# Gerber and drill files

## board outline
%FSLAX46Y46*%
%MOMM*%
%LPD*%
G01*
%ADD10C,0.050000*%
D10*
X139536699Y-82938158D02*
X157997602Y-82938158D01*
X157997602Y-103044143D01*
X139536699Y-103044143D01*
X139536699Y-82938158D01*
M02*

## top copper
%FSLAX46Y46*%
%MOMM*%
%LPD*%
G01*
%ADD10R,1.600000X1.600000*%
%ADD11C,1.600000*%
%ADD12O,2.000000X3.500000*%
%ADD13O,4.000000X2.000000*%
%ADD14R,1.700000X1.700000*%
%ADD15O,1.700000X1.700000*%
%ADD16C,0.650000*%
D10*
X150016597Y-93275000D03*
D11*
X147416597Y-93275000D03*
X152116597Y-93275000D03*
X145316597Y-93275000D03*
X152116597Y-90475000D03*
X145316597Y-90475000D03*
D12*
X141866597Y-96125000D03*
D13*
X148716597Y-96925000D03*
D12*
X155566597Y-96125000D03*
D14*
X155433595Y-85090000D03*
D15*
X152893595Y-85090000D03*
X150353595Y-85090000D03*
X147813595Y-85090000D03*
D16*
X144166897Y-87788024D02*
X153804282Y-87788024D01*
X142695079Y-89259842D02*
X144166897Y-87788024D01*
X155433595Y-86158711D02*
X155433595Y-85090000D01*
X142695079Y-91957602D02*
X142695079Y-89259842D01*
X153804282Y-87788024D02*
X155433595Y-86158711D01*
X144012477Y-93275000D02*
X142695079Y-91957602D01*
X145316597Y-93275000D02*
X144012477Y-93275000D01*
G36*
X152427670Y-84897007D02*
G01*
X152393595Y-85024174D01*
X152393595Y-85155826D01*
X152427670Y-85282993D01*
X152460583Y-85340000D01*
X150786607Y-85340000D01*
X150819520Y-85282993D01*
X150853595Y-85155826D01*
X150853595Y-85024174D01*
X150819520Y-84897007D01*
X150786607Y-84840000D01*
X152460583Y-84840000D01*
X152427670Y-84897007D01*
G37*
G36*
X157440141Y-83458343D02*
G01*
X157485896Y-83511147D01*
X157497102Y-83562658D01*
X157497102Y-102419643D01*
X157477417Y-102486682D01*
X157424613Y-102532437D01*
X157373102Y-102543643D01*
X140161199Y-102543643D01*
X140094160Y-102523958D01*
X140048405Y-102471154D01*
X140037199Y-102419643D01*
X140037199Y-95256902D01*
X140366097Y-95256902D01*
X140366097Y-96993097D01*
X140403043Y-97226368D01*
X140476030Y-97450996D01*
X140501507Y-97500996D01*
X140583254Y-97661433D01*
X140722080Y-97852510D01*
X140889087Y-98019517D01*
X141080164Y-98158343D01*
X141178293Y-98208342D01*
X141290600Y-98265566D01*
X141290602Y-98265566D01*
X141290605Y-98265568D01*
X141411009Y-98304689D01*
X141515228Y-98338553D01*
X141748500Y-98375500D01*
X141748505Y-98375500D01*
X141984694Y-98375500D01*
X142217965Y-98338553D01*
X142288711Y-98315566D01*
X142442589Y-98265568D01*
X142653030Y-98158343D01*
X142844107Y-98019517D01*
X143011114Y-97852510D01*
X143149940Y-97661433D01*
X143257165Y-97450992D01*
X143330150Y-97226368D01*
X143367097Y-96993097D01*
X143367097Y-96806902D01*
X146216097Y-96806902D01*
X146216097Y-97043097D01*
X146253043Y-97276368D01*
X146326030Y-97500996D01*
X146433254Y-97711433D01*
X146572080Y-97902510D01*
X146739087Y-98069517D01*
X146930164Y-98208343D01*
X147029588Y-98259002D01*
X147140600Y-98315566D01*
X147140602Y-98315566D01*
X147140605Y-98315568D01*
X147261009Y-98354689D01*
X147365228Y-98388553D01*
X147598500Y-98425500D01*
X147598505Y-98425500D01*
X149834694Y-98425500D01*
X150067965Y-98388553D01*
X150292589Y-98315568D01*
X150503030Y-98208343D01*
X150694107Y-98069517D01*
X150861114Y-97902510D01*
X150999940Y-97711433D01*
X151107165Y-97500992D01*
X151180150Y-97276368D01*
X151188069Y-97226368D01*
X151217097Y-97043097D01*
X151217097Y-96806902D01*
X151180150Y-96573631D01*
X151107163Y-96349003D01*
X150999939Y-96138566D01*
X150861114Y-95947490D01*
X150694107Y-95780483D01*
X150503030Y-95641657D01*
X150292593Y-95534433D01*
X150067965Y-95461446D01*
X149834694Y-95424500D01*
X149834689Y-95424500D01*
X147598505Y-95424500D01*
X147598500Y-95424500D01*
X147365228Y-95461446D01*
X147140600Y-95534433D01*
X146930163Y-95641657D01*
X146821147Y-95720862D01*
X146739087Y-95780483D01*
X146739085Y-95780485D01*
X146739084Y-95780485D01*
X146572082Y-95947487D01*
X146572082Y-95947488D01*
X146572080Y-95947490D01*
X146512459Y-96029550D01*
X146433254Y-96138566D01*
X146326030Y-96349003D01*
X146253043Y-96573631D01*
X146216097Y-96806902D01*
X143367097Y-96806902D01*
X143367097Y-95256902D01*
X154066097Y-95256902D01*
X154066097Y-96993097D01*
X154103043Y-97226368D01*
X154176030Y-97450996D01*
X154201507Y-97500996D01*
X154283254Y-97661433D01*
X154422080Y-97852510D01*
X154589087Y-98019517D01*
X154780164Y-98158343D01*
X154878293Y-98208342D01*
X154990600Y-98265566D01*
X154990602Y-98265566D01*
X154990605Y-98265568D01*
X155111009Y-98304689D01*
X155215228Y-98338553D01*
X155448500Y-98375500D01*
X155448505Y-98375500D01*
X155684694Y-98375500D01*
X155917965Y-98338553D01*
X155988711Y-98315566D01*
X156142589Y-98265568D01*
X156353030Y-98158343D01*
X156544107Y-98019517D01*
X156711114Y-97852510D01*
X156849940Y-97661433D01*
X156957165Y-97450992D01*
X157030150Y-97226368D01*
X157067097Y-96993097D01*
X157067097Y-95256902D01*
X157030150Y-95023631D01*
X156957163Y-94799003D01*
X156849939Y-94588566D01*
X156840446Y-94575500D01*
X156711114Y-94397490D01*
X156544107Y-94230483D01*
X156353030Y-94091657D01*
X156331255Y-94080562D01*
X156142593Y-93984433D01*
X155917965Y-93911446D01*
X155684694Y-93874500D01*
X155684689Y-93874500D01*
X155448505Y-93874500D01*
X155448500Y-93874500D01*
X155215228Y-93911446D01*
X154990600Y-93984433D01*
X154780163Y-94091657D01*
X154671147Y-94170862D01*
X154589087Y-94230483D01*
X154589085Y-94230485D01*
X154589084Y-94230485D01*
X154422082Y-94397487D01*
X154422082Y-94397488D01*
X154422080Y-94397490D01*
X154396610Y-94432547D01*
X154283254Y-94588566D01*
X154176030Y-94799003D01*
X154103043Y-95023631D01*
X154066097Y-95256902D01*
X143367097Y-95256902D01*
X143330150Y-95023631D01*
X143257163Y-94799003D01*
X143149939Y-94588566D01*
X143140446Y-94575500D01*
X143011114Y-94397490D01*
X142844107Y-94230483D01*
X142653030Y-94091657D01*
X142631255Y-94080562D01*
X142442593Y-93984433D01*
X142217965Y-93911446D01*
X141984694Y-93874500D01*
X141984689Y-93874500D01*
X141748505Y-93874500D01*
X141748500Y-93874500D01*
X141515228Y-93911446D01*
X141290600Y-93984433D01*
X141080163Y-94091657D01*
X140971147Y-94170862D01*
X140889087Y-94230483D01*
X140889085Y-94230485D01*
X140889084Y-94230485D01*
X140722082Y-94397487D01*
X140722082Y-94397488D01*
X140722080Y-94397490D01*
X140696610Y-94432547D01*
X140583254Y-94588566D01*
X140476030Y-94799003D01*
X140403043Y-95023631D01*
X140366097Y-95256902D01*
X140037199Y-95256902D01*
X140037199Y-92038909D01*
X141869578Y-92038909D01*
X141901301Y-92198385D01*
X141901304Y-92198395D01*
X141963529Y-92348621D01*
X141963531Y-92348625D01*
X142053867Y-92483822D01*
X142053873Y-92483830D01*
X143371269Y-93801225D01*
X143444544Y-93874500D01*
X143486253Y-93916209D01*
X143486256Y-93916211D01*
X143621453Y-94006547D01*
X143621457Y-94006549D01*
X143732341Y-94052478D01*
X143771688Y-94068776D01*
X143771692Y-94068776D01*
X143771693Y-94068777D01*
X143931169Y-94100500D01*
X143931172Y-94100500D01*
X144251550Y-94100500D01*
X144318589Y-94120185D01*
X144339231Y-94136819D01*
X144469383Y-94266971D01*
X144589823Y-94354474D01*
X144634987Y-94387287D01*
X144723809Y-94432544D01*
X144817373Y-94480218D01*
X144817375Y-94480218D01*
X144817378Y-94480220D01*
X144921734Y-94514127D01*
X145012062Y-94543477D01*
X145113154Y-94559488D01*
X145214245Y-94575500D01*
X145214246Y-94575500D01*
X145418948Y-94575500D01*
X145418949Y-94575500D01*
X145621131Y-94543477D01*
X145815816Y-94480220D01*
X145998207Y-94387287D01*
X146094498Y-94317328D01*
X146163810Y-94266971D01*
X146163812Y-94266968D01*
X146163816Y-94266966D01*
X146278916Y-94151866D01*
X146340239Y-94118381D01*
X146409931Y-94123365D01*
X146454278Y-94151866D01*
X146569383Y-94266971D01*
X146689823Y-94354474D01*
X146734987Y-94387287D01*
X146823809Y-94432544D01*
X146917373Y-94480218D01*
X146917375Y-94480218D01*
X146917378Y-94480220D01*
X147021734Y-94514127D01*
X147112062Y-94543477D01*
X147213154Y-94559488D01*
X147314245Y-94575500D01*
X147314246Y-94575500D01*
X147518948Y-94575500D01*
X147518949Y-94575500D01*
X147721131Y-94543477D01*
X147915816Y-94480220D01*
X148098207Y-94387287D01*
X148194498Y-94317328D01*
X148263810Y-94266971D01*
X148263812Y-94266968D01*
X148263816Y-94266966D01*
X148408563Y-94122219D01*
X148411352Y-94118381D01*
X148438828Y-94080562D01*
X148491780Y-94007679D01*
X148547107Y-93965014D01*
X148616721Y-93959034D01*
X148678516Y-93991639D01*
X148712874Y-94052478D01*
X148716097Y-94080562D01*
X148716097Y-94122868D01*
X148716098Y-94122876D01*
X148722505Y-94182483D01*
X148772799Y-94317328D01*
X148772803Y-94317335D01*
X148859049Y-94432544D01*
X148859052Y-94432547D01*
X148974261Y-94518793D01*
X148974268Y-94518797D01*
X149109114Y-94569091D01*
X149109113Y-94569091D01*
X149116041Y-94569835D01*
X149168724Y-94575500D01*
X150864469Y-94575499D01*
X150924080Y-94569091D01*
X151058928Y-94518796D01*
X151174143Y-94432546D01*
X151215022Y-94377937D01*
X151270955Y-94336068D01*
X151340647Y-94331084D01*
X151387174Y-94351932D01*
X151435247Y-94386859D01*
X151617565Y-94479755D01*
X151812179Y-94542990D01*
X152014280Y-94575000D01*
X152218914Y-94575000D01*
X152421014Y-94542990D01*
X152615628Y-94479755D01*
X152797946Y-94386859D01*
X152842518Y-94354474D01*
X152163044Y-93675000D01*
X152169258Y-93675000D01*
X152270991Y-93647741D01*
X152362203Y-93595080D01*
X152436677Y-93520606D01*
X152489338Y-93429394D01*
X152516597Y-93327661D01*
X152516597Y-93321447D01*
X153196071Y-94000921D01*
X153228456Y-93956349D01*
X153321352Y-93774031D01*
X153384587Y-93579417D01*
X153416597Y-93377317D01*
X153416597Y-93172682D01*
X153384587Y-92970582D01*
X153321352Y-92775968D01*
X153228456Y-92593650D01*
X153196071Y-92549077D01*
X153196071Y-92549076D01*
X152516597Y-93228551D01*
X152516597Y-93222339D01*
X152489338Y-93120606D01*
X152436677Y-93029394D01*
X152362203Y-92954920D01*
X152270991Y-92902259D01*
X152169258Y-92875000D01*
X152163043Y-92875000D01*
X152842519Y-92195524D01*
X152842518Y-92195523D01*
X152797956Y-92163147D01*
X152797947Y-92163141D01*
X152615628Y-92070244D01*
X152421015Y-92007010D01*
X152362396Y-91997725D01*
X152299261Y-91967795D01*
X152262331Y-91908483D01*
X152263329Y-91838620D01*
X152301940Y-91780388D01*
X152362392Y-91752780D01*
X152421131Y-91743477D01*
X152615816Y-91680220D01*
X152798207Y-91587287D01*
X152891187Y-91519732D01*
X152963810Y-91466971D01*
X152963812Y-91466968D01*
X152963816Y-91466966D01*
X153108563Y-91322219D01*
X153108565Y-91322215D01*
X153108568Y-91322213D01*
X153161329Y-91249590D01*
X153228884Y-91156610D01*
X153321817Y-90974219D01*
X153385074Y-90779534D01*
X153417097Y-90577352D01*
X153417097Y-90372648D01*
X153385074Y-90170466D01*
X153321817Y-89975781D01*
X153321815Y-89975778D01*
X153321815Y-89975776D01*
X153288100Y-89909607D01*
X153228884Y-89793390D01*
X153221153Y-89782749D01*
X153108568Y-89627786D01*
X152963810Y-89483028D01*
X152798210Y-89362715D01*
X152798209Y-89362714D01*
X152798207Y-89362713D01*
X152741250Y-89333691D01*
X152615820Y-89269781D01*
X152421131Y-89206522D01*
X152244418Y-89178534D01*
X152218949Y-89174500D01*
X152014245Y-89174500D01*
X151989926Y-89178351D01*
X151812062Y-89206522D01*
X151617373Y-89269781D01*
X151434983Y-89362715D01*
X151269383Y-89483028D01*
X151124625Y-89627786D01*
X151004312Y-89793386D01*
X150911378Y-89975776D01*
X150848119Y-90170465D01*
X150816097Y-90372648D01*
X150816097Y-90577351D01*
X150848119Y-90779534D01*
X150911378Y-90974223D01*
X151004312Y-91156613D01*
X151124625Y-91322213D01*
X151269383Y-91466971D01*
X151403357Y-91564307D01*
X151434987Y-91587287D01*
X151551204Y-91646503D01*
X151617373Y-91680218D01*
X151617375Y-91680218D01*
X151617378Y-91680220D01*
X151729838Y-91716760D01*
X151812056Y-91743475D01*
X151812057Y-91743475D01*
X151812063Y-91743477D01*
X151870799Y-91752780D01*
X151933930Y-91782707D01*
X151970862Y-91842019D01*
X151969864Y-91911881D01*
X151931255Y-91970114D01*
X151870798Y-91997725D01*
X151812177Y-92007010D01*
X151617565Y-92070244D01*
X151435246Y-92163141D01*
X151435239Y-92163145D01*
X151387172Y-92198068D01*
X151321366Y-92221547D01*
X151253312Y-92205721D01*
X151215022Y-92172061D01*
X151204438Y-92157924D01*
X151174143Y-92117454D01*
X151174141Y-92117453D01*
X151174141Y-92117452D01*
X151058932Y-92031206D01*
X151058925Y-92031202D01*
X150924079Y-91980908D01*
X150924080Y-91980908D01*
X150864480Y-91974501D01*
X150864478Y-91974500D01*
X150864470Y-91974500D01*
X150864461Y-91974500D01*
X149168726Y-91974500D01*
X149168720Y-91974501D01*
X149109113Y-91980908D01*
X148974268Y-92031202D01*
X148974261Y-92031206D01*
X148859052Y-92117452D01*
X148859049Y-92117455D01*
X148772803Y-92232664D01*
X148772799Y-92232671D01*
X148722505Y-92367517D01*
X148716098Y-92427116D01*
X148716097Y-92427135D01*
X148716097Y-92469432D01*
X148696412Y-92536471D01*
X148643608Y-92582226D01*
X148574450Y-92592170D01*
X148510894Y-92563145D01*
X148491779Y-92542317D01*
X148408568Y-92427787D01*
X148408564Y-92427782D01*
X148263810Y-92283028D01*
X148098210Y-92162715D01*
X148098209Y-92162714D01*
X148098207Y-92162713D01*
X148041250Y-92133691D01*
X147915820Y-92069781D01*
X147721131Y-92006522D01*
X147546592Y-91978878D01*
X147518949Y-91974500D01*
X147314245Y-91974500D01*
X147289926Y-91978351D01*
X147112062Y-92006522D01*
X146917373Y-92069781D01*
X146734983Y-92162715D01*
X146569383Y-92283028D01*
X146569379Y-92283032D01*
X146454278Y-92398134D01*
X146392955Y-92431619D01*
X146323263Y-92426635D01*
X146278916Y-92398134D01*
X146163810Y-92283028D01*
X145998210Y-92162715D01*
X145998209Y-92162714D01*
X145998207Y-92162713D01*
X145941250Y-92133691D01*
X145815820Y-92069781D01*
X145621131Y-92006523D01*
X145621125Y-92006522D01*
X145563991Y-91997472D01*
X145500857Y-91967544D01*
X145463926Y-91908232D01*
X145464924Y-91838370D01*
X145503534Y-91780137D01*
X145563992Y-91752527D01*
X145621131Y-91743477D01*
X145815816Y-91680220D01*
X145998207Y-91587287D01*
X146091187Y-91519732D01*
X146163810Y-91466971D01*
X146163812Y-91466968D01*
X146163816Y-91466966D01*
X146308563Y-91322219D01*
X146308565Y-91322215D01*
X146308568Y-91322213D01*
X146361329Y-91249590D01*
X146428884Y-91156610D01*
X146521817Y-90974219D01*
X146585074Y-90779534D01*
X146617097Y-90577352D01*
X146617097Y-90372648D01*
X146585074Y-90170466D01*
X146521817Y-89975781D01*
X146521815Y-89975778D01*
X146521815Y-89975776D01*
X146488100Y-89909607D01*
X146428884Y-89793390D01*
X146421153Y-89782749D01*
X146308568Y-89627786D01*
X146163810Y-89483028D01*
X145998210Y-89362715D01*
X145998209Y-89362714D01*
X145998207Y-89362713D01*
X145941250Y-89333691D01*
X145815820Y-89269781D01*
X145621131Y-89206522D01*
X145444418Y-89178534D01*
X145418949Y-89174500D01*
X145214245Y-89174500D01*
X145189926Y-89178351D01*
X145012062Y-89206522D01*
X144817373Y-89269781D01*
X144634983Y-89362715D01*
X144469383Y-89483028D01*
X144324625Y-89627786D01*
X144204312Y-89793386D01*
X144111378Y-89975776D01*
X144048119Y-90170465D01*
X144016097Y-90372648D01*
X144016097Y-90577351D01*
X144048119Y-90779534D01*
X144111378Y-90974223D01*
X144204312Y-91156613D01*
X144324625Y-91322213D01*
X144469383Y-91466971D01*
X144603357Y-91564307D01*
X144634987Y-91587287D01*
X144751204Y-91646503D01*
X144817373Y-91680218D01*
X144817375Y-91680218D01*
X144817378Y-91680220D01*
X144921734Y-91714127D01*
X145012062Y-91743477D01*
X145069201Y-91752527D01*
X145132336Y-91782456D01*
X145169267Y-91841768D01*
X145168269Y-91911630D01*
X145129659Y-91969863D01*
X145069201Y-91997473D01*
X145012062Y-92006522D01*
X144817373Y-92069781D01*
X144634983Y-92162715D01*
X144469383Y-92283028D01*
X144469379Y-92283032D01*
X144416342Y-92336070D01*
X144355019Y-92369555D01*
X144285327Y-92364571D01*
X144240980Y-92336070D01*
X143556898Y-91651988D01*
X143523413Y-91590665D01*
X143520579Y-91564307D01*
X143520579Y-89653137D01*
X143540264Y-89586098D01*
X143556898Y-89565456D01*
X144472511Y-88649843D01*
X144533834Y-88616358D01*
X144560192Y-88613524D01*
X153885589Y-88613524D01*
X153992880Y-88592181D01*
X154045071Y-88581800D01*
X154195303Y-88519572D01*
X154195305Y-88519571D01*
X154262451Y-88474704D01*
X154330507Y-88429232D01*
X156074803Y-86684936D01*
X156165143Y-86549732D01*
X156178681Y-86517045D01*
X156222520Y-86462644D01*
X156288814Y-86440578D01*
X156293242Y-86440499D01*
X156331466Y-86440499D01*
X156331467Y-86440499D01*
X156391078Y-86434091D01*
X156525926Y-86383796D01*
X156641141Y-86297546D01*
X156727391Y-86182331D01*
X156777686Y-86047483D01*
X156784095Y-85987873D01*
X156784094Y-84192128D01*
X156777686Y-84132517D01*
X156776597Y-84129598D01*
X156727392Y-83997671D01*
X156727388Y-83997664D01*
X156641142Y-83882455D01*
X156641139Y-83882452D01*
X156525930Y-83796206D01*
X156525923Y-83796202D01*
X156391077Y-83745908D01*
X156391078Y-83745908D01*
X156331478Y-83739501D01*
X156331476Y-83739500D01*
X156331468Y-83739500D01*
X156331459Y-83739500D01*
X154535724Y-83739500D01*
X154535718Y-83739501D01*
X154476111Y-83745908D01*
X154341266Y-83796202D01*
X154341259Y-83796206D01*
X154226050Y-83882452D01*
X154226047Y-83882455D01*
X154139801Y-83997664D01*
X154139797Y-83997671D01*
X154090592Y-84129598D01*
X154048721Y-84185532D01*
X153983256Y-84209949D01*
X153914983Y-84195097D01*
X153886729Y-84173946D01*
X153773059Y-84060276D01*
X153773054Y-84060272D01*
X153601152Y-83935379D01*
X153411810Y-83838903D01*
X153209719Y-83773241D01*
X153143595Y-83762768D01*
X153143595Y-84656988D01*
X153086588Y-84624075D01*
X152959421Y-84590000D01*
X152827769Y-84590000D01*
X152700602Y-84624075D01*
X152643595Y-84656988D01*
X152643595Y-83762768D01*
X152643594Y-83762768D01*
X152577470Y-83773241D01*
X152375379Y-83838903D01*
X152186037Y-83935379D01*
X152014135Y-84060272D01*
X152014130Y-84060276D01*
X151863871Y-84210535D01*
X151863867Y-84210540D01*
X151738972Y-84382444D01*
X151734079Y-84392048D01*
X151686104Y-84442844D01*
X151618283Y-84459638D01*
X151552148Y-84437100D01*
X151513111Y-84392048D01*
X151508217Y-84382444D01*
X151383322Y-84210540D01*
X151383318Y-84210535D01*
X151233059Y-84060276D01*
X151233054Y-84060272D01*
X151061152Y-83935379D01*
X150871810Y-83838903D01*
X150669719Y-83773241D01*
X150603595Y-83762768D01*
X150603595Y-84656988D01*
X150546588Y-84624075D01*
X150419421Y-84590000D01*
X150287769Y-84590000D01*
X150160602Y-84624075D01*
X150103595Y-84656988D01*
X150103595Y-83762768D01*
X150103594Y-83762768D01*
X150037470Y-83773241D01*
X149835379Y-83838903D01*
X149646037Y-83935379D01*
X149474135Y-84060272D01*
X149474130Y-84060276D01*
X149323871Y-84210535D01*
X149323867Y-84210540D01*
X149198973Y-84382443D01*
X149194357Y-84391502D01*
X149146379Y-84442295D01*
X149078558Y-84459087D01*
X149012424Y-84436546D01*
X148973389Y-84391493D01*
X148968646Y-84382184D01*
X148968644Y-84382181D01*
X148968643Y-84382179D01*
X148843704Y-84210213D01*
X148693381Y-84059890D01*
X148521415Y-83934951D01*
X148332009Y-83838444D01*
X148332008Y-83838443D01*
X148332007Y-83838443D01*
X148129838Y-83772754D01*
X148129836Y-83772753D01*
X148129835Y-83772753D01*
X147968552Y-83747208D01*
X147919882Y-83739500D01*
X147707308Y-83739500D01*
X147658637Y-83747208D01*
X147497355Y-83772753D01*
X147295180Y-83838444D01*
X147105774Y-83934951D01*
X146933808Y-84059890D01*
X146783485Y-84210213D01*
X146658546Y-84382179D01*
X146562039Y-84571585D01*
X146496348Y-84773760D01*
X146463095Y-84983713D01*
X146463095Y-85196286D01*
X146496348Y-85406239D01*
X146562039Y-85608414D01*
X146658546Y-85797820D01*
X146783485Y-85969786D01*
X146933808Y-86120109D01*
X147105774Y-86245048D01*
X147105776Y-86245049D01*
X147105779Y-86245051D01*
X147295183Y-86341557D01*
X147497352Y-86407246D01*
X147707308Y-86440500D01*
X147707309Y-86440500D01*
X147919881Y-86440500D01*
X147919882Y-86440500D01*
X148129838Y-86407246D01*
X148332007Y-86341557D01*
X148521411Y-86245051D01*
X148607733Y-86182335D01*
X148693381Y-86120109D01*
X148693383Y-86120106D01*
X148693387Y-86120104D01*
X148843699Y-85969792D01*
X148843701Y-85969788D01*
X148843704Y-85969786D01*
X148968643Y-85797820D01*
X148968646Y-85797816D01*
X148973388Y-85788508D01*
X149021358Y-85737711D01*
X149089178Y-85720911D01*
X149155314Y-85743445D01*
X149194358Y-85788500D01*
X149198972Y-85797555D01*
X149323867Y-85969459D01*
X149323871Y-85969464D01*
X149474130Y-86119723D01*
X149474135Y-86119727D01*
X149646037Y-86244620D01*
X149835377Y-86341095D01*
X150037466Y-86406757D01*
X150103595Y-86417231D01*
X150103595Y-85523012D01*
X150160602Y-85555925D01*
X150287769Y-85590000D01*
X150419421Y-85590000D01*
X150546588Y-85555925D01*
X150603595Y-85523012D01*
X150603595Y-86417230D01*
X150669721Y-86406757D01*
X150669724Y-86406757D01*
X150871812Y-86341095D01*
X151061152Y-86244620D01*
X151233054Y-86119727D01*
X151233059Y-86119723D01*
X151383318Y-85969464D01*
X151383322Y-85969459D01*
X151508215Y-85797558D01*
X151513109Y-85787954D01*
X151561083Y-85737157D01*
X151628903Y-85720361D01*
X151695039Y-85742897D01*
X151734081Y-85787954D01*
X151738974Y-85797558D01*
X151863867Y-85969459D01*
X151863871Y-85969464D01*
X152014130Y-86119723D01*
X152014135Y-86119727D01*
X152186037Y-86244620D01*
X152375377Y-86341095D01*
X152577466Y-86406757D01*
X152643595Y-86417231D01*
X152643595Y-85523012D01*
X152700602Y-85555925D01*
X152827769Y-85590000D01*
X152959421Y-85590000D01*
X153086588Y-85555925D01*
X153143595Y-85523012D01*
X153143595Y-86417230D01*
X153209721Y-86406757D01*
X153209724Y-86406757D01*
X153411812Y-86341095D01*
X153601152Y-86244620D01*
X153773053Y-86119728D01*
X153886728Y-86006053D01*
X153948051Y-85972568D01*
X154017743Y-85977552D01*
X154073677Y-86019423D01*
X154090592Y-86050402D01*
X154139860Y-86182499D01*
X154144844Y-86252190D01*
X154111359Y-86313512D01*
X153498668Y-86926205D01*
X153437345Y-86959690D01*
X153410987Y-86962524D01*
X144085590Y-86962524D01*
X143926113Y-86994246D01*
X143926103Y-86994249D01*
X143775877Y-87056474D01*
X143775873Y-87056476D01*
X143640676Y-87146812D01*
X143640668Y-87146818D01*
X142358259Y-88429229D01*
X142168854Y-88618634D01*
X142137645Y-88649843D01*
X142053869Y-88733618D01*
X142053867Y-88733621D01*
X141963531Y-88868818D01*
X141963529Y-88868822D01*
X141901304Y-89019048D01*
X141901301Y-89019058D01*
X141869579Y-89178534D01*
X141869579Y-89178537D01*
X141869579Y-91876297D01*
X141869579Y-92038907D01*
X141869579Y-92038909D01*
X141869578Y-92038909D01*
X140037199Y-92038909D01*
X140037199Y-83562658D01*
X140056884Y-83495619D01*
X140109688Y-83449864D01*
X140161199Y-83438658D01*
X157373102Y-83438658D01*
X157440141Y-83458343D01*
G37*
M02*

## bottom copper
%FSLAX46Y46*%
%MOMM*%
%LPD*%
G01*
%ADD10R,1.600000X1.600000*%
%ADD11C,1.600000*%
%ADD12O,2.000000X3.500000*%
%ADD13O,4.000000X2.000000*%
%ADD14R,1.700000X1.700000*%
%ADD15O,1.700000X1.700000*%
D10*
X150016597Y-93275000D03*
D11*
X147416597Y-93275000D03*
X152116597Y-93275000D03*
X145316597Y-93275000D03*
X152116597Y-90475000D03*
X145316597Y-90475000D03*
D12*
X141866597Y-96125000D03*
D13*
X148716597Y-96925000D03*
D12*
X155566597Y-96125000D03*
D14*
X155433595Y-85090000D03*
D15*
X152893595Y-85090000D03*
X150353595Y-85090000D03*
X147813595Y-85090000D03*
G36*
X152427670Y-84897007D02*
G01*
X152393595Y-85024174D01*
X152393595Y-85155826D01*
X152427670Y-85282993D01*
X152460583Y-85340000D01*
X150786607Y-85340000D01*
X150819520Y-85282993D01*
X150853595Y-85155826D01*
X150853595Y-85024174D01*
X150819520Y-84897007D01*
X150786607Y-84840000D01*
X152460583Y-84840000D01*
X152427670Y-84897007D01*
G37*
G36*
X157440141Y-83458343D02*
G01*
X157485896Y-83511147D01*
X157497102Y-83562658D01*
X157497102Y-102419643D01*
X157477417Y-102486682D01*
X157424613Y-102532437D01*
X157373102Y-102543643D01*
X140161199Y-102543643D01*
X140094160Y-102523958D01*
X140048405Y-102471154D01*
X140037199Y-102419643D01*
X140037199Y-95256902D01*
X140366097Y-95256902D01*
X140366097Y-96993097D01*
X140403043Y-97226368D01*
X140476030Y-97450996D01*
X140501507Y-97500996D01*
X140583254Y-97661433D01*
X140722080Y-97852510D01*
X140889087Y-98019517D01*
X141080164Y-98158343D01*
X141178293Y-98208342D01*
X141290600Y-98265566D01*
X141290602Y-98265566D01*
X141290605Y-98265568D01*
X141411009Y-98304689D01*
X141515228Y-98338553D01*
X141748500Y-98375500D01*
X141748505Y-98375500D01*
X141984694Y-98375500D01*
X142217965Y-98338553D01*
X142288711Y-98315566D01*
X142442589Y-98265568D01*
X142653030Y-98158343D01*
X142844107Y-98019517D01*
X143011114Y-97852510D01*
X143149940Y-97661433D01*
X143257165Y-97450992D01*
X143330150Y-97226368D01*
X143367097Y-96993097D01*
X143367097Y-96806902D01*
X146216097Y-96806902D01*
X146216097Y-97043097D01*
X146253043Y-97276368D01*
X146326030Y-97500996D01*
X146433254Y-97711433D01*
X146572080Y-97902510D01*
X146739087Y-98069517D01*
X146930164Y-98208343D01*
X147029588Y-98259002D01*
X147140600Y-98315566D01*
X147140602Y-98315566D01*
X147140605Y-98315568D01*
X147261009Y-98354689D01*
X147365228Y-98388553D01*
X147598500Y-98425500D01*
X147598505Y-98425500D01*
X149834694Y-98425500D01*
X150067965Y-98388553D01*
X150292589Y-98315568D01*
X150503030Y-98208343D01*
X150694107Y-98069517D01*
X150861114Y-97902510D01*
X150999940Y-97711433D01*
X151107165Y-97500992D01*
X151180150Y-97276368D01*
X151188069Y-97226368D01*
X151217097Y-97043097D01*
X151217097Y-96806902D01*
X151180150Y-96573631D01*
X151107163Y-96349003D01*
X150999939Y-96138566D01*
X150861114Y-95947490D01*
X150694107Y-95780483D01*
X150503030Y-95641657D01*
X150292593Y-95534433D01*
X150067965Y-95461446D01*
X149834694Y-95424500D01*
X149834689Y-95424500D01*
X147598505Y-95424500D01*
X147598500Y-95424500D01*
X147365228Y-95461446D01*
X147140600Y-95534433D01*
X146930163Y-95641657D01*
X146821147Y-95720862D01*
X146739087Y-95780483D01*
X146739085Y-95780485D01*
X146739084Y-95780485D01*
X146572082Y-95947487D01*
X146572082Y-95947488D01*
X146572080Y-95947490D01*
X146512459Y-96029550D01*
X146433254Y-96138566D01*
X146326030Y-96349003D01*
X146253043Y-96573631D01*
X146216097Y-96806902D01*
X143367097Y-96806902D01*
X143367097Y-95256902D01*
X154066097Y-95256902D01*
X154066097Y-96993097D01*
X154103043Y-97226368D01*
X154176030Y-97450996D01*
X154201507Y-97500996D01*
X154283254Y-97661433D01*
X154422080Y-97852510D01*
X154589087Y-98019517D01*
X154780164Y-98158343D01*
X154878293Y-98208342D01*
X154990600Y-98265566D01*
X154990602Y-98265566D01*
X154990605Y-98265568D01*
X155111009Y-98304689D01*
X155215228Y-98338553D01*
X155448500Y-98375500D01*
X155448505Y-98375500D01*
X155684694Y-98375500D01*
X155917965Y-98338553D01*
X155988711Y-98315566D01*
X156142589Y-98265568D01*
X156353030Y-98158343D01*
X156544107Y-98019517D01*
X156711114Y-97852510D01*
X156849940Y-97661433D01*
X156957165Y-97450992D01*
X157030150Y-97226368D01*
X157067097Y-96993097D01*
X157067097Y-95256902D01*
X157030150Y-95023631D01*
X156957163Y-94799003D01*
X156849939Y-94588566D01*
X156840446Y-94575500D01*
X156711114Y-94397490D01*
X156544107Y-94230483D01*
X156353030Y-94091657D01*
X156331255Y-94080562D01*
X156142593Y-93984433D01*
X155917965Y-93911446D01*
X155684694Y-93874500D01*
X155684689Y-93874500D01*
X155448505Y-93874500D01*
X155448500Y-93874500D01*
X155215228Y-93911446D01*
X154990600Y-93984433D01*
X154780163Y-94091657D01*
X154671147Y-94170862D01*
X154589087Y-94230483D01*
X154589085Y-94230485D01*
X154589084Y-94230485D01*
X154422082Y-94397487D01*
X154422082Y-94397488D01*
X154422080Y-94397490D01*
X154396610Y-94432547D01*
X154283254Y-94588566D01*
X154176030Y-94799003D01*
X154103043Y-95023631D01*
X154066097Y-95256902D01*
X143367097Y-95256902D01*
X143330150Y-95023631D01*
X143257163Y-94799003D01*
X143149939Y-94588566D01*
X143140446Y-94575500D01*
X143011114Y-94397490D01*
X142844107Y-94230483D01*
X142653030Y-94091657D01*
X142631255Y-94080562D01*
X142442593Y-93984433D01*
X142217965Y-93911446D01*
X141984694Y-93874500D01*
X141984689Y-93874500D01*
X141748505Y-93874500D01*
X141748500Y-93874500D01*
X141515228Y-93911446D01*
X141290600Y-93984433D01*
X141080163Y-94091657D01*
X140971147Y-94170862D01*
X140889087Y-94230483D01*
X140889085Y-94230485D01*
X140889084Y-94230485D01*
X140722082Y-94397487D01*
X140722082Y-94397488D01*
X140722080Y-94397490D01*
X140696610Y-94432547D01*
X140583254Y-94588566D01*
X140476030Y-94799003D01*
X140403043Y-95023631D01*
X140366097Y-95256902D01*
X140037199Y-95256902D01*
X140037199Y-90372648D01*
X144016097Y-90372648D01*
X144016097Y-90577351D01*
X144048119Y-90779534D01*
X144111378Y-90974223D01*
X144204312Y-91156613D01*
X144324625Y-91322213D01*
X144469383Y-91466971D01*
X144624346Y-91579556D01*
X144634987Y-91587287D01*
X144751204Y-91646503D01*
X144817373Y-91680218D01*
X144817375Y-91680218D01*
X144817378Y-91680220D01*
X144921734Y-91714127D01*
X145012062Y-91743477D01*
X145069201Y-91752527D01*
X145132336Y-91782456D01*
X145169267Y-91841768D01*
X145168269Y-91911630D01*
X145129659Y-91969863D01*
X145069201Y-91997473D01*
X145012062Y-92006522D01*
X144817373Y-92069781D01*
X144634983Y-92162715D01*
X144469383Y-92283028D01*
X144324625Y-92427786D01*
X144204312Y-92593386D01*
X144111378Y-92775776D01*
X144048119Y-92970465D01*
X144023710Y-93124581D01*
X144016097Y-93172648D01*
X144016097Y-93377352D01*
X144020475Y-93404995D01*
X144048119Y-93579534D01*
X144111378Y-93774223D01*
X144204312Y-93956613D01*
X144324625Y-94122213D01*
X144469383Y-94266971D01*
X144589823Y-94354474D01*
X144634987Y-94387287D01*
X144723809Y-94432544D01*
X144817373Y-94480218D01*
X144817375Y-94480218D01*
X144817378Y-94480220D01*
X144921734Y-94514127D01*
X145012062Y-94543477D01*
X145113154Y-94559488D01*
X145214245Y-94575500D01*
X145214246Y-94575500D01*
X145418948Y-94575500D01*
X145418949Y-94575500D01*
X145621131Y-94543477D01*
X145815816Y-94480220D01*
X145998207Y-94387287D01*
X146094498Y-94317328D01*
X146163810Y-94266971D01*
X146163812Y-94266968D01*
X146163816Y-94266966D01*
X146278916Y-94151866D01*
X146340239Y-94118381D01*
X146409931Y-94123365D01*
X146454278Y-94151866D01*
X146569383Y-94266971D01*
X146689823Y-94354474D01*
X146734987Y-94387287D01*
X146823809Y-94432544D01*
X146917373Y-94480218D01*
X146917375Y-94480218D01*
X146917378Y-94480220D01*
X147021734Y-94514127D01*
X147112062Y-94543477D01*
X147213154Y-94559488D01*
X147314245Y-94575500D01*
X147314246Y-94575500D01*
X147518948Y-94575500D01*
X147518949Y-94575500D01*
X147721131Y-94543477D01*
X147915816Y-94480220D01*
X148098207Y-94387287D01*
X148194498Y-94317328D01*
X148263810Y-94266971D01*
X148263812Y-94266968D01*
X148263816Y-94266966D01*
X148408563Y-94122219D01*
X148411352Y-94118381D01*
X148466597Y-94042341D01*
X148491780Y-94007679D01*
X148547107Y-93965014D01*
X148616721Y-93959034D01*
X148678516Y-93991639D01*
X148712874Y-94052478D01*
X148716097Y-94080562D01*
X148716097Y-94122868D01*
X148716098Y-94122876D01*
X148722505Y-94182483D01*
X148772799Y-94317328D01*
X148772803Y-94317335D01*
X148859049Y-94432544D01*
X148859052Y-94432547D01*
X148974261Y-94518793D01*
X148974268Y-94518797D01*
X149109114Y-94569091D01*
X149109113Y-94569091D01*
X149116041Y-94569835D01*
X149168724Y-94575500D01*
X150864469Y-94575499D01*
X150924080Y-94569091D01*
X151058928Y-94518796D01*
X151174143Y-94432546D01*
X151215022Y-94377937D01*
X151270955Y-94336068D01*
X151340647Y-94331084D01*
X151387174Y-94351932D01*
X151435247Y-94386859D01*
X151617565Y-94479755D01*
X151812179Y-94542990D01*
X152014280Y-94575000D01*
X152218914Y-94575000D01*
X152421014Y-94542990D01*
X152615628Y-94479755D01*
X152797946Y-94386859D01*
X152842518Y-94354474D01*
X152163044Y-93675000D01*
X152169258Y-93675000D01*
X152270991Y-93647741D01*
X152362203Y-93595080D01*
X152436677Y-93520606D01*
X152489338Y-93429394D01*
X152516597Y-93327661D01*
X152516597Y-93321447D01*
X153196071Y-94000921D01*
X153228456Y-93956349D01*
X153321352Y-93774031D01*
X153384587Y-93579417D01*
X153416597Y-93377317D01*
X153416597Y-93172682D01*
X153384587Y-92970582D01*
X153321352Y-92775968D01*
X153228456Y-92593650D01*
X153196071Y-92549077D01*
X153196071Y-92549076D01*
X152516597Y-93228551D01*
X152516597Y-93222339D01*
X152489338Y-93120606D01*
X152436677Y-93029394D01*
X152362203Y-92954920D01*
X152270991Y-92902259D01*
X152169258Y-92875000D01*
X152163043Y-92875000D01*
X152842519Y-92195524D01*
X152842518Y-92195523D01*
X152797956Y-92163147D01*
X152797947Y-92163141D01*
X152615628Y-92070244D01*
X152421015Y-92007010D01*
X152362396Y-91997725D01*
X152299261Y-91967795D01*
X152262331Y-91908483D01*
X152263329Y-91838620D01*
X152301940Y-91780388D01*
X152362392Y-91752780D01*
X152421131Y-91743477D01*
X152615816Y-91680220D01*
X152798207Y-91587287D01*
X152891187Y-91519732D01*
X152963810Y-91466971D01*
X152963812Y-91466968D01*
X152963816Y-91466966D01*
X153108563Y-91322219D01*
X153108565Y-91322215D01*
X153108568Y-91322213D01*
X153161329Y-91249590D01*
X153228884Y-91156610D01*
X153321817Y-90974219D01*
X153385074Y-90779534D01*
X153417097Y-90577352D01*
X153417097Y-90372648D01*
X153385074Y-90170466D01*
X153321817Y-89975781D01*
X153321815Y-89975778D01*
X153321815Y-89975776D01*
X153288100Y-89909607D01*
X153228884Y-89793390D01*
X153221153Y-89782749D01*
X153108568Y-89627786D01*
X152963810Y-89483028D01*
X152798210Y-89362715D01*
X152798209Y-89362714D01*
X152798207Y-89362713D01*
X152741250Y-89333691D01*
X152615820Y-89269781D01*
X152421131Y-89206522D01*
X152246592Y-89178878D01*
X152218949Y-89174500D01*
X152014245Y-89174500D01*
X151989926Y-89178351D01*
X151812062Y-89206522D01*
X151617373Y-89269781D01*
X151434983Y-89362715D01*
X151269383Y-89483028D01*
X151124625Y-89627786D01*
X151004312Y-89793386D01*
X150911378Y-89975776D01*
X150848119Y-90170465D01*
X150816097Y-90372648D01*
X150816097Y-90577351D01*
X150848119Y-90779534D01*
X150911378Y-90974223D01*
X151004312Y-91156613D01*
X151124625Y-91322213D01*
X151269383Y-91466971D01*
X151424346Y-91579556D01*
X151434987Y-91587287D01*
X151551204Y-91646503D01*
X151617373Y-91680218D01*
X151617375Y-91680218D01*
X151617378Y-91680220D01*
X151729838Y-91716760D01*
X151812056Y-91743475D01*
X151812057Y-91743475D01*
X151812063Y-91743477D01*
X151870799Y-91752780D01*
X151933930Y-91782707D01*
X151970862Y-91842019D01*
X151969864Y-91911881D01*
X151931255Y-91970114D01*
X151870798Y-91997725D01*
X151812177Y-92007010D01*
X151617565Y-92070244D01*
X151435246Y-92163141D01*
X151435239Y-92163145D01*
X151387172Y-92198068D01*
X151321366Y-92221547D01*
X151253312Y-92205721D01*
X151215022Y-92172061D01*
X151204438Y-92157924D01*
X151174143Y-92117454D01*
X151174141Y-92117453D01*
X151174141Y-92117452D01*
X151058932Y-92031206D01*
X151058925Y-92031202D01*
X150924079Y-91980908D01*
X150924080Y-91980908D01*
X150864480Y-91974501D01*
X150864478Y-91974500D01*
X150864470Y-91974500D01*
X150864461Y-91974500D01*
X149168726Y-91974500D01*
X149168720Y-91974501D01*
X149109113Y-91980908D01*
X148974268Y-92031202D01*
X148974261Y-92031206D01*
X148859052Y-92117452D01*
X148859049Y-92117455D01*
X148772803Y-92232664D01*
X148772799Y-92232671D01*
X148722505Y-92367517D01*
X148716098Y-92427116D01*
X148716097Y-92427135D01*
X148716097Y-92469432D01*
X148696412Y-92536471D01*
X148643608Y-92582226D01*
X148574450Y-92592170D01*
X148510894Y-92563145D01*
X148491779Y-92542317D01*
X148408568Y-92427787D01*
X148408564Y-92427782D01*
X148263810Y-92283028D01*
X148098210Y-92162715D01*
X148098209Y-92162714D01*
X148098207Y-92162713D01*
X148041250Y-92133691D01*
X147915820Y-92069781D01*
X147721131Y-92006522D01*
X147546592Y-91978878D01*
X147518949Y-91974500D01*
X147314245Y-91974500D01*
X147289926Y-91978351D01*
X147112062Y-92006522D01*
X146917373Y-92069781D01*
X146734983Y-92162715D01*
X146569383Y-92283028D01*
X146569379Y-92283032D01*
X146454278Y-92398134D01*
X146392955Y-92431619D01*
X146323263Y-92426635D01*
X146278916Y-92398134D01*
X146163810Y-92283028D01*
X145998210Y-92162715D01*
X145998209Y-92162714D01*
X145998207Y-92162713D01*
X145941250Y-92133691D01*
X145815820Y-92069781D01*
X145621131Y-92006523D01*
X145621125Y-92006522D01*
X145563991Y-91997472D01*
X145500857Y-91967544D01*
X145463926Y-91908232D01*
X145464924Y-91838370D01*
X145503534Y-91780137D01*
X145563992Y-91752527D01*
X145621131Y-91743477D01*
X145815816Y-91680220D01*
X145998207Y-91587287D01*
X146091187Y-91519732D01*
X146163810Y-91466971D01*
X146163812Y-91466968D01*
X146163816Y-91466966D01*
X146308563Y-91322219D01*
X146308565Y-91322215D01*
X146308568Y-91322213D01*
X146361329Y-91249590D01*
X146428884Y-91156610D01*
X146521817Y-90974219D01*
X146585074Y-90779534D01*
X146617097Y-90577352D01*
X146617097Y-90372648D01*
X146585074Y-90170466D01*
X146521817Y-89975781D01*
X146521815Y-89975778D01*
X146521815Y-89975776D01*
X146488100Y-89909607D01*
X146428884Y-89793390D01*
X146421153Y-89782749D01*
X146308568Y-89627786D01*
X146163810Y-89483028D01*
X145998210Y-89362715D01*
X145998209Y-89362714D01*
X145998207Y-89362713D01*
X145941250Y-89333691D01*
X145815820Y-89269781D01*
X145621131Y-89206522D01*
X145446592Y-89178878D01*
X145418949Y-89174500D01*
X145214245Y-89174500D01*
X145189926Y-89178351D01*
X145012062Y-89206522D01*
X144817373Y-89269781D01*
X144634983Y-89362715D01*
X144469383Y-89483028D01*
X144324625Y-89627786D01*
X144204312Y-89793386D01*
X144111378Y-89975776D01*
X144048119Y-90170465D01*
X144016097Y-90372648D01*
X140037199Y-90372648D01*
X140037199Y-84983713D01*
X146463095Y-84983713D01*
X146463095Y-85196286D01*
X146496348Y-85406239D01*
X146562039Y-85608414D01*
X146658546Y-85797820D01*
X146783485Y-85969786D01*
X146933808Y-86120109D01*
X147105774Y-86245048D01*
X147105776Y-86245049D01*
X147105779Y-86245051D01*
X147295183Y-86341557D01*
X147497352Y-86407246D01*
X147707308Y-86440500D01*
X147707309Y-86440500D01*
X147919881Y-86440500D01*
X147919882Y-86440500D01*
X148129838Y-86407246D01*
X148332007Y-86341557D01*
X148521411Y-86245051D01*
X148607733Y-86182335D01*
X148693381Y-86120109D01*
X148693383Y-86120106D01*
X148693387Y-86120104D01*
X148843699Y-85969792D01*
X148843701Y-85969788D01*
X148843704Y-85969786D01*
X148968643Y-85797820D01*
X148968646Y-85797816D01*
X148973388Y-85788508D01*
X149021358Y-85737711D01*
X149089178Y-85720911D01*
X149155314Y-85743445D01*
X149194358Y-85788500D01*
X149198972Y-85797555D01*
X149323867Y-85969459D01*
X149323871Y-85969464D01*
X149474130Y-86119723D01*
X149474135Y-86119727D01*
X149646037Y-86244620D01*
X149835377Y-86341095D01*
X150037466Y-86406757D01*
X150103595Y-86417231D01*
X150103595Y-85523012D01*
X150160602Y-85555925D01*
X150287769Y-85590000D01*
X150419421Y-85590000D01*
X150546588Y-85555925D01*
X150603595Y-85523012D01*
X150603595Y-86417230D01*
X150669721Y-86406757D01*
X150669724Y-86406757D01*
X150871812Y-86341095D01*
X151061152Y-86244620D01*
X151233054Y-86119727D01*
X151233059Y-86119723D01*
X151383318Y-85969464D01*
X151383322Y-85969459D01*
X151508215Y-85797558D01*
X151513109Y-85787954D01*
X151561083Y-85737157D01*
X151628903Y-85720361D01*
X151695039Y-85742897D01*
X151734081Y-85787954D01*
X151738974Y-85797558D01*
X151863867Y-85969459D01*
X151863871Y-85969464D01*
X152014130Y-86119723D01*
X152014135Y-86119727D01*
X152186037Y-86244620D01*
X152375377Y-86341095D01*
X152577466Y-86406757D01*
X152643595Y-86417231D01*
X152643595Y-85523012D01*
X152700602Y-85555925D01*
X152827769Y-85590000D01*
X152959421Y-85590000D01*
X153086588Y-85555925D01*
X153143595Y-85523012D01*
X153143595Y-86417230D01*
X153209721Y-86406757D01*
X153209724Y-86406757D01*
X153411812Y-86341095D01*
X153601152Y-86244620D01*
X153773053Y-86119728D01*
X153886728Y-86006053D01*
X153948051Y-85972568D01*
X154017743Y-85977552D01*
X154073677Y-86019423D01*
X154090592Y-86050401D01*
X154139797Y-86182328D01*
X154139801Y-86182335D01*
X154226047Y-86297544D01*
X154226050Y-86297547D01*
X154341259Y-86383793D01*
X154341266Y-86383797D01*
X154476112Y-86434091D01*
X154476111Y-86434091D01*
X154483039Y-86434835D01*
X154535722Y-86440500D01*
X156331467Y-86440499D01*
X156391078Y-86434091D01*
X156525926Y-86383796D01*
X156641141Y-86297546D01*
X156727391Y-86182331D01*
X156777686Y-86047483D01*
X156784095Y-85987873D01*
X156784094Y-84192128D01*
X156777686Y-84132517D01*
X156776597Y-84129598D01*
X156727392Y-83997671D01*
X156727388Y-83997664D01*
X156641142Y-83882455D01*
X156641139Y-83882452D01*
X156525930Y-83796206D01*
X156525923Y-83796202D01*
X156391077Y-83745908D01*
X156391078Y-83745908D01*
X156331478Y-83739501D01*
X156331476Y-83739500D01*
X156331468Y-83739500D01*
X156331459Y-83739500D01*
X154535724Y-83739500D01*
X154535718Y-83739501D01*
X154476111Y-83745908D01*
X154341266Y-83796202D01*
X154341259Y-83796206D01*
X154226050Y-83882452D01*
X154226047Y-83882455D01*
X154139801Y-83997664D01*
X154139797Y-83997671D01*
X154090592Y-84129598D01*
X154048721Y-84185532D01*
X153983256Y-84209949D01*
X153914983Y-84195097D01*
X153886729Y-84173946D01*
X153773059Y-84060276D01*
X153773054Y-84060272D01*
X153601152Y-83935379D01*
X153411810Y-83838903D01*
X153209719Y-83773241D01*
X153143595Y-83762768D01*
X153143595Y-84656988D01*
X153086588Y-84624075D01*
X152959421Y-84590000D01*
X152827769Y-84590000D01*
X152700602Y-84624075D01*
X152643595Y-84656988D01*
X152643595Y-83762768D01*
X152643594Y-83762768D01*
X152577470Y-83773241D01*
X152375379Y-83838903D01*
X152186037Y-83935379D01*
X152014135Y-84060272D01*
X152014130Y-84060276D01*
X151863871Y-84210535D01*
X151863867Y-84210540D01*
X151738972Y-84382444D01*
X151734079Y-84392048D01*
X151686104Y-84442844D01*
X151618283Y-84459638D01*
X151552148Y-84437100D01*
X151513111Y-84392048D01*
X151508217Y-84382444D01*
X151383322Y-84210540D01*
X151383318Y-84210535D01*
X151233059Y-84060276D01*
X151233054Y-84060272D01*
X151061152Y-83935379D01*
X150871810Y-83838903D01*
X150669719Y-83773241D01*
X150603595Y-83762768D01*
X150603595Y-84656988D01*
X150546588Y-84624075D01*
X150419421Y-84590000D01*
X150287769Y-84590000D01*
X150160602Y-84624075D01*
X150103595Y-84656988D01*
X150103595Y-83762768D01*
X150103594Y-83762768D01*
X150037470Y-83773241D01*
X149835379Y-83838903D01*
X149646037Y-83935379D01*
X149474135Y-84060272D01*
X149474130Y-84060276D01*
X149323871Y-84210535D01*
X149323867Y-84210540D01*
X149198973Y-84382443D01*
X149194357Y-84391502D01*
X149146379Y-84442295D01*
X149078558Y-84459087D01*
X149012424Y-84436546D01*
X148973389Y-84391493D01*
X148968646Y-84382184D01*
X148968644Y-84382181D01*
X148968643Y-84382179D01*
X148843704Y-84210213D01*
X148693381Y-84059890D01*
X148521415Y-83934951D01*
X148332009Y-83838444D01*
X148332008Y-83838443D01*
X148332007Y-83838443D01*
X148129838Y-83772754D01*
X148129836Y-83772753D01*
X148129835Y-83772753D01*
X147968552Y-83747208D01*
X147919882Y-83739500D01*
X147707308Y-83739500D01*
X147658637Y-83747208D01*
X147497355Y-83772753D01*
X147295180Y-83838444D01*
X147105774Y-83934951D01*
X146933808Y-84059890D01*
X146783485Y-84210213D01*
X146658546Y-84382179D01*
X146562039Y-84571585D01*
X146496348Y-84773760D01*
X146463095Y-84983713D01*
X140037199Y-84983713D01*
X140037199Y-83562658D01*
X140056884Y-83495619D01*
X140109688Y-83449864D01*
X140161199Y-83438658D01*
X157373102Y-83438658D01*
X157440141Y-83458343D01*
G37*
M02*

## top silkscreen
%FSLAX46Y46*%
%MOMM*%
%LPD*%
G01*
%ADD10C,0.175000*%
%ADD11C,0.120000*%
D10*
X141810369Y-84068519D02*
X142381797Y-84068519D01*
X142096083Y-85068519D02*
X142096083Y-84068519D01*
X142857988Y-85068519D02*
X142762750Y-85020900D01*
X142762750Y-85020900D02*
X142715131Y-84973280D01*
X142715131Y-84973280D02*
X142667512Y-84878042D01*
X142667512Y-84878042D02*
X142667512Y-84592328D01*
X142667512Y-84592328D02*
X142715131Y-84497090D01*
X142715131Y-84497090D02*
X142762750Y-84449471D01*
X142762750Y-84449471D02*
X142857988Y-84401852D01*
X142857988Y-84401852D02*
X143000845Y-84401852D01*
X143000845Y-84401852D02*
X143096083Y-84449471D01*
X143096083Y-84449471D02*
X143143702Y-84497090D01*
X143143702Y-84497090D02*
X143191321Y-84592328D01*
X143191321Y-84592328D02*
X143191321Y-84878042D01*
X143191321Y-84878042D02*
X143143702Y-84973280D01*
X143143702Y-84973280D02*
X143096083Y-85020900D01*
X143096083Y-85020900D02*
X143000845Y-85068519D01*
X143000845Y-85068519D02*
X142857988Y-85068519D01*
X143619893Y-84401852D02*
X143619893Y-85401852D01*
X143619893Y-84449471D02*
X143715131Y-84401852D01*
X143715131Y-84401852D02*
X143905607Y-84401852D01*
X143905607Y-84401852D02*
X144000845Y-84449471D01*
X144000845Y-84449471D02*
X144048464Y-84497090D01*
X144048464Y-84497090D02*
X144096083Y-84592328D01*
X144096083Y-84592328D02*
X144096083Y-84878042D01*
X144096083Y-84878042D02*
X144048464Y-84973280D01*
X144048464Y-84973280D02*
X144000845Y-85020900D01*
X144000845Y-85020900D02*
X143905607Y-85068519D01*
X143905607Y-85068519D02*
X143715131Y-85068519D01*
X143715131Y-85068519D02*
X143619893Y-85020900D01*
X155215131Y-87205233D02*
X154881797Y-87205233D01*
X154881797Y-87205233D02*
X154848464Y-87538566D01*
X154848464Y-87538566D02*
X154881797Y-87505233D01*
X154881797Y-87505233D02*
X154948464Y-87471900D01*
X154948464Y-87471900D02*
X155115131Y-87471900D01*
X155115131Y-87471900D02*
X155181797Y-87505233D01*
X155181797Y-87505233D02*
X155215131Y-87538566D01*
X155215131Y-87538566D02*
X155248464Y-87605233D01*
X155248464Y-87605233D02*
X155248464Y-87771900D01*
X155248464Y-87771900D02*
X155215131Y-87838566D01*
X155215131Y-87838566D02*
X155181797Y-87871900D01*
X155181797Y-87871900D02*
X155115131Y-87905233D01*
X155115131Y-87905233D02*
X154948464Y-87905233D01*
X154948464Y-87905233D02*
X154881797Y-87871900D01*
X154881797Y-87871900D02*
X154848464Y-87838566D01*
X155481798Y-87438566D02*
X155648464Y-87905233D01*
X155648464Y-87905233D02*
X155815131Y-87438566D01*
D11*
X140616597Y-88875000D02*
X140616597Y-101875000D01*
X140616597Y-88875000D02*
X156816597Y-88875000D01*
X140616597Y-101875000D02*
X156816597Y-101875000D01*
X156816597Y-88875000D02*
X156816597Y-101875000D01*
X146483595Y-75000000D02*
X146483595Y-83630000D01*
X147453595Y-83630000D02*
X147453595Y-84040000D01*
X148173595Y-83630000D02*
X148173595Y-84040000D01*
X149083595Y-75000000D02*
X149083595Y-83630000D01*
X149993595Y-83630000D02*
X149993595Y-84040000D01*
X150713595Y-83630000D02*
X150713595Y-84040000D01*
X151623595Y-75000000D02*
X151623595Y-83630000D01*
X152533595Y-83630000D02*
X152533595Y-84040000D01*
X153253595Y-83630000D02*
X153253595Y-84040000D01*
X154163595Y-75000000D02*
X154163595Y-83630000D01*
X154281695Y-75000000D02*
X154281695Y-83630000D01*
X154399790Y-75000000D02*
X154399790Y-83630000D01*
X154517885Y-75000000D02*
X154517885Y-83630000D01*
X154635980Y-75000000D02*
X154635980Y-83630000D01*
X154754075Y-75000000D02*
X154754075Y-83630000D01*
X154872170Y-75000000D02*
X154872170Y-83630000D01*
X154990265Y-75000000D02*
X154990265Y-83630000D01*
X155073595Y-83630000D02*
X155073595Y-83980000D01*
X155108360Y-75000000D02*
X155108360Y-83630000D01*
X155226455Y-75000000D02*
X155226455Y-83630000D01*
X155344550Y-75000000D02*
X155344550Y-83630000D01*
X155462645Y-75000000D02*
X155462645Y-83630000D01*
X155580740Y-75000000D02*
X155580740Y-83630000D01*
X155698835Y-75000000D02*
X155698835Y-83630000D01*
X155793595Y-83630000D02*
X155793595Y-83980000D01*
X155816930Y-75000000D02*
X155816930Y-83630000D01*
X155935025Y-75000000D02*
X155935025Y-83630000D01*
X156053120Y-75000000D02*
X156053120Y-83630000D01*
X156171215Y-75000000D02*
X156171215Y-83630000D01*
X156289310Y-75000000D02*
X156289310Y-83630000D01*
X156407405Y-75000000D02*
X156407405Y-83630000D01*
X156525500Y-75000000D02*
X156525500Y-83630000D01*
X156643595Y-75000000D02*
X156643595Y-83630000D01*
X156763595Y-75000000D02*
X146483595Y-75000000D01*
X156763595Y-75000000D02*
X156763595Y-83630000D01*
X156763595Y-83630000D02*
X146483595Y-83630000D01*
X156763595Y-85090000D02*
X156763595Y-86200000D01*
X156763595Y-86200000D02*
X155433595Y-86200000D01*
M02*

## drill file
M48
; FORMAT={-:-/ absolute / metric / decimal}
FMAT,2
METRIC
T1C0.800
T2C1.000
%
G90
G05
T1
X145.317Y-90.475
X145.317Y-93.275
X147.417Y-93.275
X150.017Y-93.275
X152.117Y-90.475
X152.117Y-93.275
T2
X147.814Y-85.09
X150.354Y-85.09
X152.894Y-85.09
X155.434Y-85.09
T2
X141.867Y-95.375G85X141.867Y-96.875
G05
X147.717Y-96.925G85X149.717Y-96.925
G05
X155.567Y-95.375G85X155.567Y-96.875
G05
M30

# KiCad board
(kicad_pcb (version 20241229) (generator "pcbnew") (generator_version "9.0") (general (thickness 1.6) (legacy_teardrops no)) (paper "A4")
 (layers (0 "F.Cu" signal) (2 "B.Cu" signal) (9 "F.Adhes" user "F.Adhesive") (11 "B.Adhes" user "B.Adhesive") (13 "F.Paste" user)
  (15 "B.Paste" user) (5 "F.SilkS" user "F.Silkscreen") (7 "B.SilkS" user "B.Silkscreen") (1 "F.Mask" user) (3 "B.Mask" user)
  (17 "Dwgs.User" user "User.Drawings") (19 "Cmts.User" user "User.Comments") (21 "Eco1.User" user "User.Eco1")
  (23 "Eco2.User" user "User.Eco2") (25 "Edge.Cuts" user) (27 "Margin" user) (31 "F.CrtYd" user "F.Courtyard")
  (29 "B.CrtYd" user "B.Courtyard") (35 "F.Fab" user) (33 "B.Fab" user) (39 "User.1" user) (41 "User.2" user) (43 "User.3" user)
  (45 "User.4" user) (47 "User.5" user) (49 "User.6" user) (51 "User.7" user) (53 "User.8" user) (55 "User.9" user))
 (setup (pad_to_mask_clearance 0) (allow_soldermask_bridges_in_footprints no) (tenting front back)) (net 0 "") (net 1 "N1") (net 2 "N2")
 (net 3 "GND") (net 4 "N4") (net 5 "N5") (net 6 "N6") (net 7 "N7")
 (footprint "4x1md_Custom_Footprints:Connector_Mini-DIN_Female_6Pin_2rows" (layer "F.Cu") (at 150.016597 93.275)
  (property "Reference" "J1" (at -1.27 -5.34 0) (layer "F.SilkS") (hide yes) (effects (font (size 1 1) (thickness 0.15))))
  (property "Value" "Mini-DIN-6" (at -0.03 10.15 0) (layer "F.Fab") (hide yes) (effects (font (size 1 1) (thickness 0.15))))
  (fp_line (start -9.4 -4.4) (end -9.4 8.6) (stroke (width 0.12) (type solid)) (layer "F.SilkS"))
  (fp_line (start -9.4 -4.4) (end 6.8 -4.4) (stroke (width 0.12) (type solid)) (layer "F.SilkS"))
  (fp_line (start -9.4 8.6) (end 6.8 8.6) (stroke (width 0.12) (type solid)) (layer "F.SilkS"))
  (fp_line (start 6.8 -4.4) (end 6.8 8.6) (stroke (width 0.12) (type solid)) (layer "F.SilkS"))
  (pad "1" thru_hole rect (at 0 0) (size 1.6 1.6) (drill 0.8) (layers "*.Cu" "*.Mask") (remove_unused_layers no) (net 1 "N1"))
  (pad "2" thru_hole circle (at -2.6 0) (size 1.6 1.6) (drill 0.8) (layers "*.Cu" "*.Mask") (remove_unused_layers no) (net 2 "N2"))
  (pad "3" thru_hole circle (at 2.1 0) (size 1.6 1.6) (drill 0.8) (layers "*.Cu" "*.Mask") (remove_unused_layers no) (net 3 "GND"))
  (pad "4" thru_hole circle (at -4.7 0) (size 1.6 1.6) (drill 0.8) (layers "*.Cu" "*.Mask") (remove_unused_layers no) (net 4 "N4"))
  (pad "5" thru_hole circle (at 2.1 -2.8) (size 1.6 1.6) (drill 0.8) (layers "*.Cu" "*.Mask") (remove_unused_layers no) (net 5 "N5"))
  (pad "6" thru_hole circle (at -4.7 -2.8) (size 1.6 1.6) (drill 0.8) (layers "*.Cu" "*.Mask") (remove_unused_layers no) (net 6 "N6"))
  (pad "7" thru_hole oval (at -8.15 2.85) (size 2 3.5) (drill oval 1 2.5) (layers "*.Cu" "*.Mask") (remove_unused_layers no))
  (pad "7" thru_hole oval (at -1.3 3.65) (size 4 2) (drill oval 3 1) (layers "*.Cu" "*.Mask") (remove_unused_layers no))
  (pad "7" thru_hole oval (at 5.55 2.85) (size 2 3.5) (drill oval 1 2.5) (layers "*.Cu" "*.Mask") (remove_unused_layers no)))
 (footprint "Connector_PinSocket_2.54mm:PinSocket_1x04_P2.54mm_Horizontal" (layer "F.Cu") (at 155.433595 85.09 -90)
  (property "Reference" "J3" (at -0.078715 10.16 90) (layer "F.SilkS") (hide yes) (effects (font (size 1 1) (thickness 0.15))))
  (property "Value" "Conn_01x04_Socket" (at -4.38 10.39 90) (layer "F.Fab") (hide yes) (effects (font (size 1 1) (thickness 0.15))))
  (fp_line (start -10.09 8.95) (end -1.46 8.95) (stroke (width 0.12) (type solid)) (layer "F.SilkS"))
  (fp_line (start -1.46 7.98) (end -1.05 7.98) (stroke (width 0.12) (type solid)) (layer "F.SilkS"))
  (fp_line (start -1.46 7.26) (end -1.05 7.26) (stroke (width 0.12) (type solid)) (layer "F.SilkS"))
  (fp_line (start -10.09 6.35) (end -1.46 6.35) (stroke (width 0.12) (type solid)) (layer "F.SilkS"))
  (fp_line (start -1.46 5.44) (end -1.05 5.44) (stroke (width 0.12) (type solid)) (layer "F.SilkS"))
  (fp_line (start -1.46 4.72) (end -1.05 4.72) (stroke (width 0.12) (type solid)) (layer "F.SilkS"))
  (fp_line (start -10.09 3.81) (end -1.46 3.81) (stroke (width 0.12) (type solid)) (layer "F.SilkS"))
  (fp_line (start -1.46 2.9) (end -1.05 2.9) (stroke (width 0.12) (type solid)) (layer "F.SilkS"))
  (fp_line (start -1.46 2.18) (end -1.05 2.18) (stroke (width 0.12) (type solid)) (layer "F.SilkS"))
  (fp_line (start -10.09 1.27) (end -1.46 1.27) (stroke (width 0.12) (type solid)) (layer "F.SilkS"))
  (fp_line (start -10.09 1.1519) (end -1.46 1.1519) (stroke (width 0.12) (type solid)) (layer "F.SilkS"))
  (fp_line (start -10.09 1.033805) (end -1.46 1.033805) (stroke (width 0.12) (type solid)) (layer "F.SilkS"))
  (fp_line (start -10.09 0.91571) (end -1.46 0.91571) (stroke (width 0.12) (type solid)) (layer "F.SilkS"))
  (fp_line (start -10.09 0.797615) (end -1.46 0.797615) (stroke (width 0.12) (type solid)) (layer "F.SilkS"))
  (fp_line (start -10.09 0.67952) (end -1.46 0.67952) (stroke (width 0.12) (type solid)) (layer "F.SilkS"))
  (fp_line (start -10.09 0.561425) (end -1.46 0.561425) (stroke (width 0.12) (type solid)) (layer "F.SilkS"))
  (fp_line (start -10.09 0.44333) (end -1.46 0.44333) (stroke (width 0.12) (type solid)) (layer "F.SilkS"))
  (fp_line (start -1.46 0.36) (end -1.11 0.36) (stroke (width 0.12) (type solid)) (layer "F.SilkS"))
  (fp_line (start -10.09 0.325235) (end -1.46 0.325235) (stroke (width 0.12) (type solid)) (layer "F.SilkS"))
  (fp_line (start -10.09 0.20714) (end -1.46 0.20714) (stroke (width 0.12) (type solid)) (layer "F.SilkS"))
  (fp_line (start -10.09 0.089045) (end -1.46 0.089045) (stroke (width 0.12) (type solid)) (layer "F.SilkS"))
  (fp_line (start -10.09 -0.02905) (end -1.46 -0.02905) (stroke (width 0.12) (type solid)) (layer "F.SilkS"))
  (fp_line (start -10.09 -0.147145) (end -1.46 -0.147145) (stroke (width 0.12) (type solid)) (layer "F.SilkS"))
  (fp_line (start -10.09 -0.26524) (end -1.46 -0.26524) (stroke (width 0.12) (type solid)) (layer "F.SilkS"))
  (fp_line (start -1.46 -0.36) (end -1.11 -0.36) (stroke (width 0.12) (type solid)) (layer "F.SilkS"))
  (fp_line (start -10.09 -0.383335) (end -1.46 -0.383335) (stroke (width 0.12) (type solid)) (layer "F.SilkS"))
  (fp_line (start -10.09 -0.50143) (end -1.46 -0.50143) (stroke (width 0.12) (type solid)) (layer "F.SilkS"))
  (fp_line (start -10.09 -0.619525) (end -1.46 -0.619525) (stroke (width 0.12) (type solid)) (layer "F.SilkS"))
  (fp_line (start -10.09 -0.73762) (end -1.46 -0.73762) (stroke (width 0.12) (type solid)) (layer "F.SilkS"))
  (fp_line (start -10.09 -0.855715) (end -1.46 -0.855715) (stroke (width 0.12) (type solid)) (layer "F.SilkS"))
  (fp_line (start -10.09 -0.97381) (end -1.46 -0.97381) (stroke (width 0.12) (type solid)) (layer "F.SilkS"))
  (fp_line (start -10.09 -1.091905) (end -1.46 -1.091905) (stroke (width 0.12) (type solid)) (layer "F.SilkS"))
  (fp_line (start -10.09 -1.21) (end -1.46 -1.21) (stroke (width 0.12) (type solid)) (layer "F.SilkS"))
  (fp_line (start -10.09 -1.33) (end -10.09 8.95) (stroke (width 0.12) (type solid)) (layer "F.SilkS"))
  (fp_line (start -10.09 -1.33) (end -1.46 -1.33) (stroke (width 0.12) (type solid)) (layer "F.SilkS"))
  (fp_line (start -1.46 -1.33) (end -1.46 8.95) (stroke (width 0.12) (type solid)) (layer "F.SilkS"))
  (fp_line (start 0 -1.33) (end 1.11 -1.33) (stroke (width 0.12) (type solid)) (layer "F.SilkS"))
  (fp_line (start 1.11 -1.33) (end 1.11 0) (stroke (width 0.12) (type solid)) (layer "F.SilkS"))
  (pad "1" thru_hole rect (at 0 0 270) (size 1.7 1.7) (drill 1) (layers "*.Cu" "*.Mask") (remove_unused_layers no) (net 4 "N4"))
  (pad "2" thru_hole oval (at 0 2.54 270) (size 1.7 1.7) (drill 1) (layers "*.Cu" "*.Mask") (remove_unused_layers no) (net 3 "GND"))
  (pad "3" thru_hole oval (at 0 5.08 270) (size 1.7 1.7) (drill 1) (layers "*.Cu" "*.Mask") (remove_unused_layers no) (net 3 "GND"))
  (pad "4" thru_hole oval (at 0 7.62 270) (size 1.7 1.7) (drill 1) (layers "*.Cu" "*.Mask") (remove_unused_layers no) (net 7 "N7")))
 (gr_rect (start 139.536699 82.938158) (end 157.997602 103.044143) (stroke (width 0.05) (type default)) (fill no) (layer "Edge.Cuts"))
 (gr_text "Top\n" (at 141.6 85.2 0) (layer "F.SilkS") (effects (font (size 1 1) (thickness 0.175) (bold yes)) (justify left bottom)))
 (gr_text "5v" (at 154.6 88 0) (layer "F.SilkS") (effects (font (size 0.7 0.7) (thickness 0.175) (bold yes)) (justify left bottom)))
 (segment (start 144.166897 87.788024) (end 153.804282 87.788024) (width 0.65) (layer "F.Cu") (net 4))
 (segment (start 142.695079 89.259842) (end 144.166897 87.788024) (width 0.65) (layer "F.Cu") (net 4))
 (segment (start 155.433595 86.158711) (end 155.433595 85.09) (width 0.65) (layer "F.Cu") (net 4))
 (segment (start 142.695079 91.957602) (end 142.695079 89.259842) (width 0.65) (layer "F.Cu") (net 4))
 (segment (start 153.804282 87.788024) (end 155.433595 86.158711) (width 0.65) (layer "F.Cu") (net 4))
 (segment (start 144.012477 93.275) (end 142.695079 91.957602) (width 0.65) (layer "F.Cu") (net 4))
 (segment (start 145.316597 93.275) (end 144.012477 93.275) (width 0.65) (layer "F.Cu") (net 4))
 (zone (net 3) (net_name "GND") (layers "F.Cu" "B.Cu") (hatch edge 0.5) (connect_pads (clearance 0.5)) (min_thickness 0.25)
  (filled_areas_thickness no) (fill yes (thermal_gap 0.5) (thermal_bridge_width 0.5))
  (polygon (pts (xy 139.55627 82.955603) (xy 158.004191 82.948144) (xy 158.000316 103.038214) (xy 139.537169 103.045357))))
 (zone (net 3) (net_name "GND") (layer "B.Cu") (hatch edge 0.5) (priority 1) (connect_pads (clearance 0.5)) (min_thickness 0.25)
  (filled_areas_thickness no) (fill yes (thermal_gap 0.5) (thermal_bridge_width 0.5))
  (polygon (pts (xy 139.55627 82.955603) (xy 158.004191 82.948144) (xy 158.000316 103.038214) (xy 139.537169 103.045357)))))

